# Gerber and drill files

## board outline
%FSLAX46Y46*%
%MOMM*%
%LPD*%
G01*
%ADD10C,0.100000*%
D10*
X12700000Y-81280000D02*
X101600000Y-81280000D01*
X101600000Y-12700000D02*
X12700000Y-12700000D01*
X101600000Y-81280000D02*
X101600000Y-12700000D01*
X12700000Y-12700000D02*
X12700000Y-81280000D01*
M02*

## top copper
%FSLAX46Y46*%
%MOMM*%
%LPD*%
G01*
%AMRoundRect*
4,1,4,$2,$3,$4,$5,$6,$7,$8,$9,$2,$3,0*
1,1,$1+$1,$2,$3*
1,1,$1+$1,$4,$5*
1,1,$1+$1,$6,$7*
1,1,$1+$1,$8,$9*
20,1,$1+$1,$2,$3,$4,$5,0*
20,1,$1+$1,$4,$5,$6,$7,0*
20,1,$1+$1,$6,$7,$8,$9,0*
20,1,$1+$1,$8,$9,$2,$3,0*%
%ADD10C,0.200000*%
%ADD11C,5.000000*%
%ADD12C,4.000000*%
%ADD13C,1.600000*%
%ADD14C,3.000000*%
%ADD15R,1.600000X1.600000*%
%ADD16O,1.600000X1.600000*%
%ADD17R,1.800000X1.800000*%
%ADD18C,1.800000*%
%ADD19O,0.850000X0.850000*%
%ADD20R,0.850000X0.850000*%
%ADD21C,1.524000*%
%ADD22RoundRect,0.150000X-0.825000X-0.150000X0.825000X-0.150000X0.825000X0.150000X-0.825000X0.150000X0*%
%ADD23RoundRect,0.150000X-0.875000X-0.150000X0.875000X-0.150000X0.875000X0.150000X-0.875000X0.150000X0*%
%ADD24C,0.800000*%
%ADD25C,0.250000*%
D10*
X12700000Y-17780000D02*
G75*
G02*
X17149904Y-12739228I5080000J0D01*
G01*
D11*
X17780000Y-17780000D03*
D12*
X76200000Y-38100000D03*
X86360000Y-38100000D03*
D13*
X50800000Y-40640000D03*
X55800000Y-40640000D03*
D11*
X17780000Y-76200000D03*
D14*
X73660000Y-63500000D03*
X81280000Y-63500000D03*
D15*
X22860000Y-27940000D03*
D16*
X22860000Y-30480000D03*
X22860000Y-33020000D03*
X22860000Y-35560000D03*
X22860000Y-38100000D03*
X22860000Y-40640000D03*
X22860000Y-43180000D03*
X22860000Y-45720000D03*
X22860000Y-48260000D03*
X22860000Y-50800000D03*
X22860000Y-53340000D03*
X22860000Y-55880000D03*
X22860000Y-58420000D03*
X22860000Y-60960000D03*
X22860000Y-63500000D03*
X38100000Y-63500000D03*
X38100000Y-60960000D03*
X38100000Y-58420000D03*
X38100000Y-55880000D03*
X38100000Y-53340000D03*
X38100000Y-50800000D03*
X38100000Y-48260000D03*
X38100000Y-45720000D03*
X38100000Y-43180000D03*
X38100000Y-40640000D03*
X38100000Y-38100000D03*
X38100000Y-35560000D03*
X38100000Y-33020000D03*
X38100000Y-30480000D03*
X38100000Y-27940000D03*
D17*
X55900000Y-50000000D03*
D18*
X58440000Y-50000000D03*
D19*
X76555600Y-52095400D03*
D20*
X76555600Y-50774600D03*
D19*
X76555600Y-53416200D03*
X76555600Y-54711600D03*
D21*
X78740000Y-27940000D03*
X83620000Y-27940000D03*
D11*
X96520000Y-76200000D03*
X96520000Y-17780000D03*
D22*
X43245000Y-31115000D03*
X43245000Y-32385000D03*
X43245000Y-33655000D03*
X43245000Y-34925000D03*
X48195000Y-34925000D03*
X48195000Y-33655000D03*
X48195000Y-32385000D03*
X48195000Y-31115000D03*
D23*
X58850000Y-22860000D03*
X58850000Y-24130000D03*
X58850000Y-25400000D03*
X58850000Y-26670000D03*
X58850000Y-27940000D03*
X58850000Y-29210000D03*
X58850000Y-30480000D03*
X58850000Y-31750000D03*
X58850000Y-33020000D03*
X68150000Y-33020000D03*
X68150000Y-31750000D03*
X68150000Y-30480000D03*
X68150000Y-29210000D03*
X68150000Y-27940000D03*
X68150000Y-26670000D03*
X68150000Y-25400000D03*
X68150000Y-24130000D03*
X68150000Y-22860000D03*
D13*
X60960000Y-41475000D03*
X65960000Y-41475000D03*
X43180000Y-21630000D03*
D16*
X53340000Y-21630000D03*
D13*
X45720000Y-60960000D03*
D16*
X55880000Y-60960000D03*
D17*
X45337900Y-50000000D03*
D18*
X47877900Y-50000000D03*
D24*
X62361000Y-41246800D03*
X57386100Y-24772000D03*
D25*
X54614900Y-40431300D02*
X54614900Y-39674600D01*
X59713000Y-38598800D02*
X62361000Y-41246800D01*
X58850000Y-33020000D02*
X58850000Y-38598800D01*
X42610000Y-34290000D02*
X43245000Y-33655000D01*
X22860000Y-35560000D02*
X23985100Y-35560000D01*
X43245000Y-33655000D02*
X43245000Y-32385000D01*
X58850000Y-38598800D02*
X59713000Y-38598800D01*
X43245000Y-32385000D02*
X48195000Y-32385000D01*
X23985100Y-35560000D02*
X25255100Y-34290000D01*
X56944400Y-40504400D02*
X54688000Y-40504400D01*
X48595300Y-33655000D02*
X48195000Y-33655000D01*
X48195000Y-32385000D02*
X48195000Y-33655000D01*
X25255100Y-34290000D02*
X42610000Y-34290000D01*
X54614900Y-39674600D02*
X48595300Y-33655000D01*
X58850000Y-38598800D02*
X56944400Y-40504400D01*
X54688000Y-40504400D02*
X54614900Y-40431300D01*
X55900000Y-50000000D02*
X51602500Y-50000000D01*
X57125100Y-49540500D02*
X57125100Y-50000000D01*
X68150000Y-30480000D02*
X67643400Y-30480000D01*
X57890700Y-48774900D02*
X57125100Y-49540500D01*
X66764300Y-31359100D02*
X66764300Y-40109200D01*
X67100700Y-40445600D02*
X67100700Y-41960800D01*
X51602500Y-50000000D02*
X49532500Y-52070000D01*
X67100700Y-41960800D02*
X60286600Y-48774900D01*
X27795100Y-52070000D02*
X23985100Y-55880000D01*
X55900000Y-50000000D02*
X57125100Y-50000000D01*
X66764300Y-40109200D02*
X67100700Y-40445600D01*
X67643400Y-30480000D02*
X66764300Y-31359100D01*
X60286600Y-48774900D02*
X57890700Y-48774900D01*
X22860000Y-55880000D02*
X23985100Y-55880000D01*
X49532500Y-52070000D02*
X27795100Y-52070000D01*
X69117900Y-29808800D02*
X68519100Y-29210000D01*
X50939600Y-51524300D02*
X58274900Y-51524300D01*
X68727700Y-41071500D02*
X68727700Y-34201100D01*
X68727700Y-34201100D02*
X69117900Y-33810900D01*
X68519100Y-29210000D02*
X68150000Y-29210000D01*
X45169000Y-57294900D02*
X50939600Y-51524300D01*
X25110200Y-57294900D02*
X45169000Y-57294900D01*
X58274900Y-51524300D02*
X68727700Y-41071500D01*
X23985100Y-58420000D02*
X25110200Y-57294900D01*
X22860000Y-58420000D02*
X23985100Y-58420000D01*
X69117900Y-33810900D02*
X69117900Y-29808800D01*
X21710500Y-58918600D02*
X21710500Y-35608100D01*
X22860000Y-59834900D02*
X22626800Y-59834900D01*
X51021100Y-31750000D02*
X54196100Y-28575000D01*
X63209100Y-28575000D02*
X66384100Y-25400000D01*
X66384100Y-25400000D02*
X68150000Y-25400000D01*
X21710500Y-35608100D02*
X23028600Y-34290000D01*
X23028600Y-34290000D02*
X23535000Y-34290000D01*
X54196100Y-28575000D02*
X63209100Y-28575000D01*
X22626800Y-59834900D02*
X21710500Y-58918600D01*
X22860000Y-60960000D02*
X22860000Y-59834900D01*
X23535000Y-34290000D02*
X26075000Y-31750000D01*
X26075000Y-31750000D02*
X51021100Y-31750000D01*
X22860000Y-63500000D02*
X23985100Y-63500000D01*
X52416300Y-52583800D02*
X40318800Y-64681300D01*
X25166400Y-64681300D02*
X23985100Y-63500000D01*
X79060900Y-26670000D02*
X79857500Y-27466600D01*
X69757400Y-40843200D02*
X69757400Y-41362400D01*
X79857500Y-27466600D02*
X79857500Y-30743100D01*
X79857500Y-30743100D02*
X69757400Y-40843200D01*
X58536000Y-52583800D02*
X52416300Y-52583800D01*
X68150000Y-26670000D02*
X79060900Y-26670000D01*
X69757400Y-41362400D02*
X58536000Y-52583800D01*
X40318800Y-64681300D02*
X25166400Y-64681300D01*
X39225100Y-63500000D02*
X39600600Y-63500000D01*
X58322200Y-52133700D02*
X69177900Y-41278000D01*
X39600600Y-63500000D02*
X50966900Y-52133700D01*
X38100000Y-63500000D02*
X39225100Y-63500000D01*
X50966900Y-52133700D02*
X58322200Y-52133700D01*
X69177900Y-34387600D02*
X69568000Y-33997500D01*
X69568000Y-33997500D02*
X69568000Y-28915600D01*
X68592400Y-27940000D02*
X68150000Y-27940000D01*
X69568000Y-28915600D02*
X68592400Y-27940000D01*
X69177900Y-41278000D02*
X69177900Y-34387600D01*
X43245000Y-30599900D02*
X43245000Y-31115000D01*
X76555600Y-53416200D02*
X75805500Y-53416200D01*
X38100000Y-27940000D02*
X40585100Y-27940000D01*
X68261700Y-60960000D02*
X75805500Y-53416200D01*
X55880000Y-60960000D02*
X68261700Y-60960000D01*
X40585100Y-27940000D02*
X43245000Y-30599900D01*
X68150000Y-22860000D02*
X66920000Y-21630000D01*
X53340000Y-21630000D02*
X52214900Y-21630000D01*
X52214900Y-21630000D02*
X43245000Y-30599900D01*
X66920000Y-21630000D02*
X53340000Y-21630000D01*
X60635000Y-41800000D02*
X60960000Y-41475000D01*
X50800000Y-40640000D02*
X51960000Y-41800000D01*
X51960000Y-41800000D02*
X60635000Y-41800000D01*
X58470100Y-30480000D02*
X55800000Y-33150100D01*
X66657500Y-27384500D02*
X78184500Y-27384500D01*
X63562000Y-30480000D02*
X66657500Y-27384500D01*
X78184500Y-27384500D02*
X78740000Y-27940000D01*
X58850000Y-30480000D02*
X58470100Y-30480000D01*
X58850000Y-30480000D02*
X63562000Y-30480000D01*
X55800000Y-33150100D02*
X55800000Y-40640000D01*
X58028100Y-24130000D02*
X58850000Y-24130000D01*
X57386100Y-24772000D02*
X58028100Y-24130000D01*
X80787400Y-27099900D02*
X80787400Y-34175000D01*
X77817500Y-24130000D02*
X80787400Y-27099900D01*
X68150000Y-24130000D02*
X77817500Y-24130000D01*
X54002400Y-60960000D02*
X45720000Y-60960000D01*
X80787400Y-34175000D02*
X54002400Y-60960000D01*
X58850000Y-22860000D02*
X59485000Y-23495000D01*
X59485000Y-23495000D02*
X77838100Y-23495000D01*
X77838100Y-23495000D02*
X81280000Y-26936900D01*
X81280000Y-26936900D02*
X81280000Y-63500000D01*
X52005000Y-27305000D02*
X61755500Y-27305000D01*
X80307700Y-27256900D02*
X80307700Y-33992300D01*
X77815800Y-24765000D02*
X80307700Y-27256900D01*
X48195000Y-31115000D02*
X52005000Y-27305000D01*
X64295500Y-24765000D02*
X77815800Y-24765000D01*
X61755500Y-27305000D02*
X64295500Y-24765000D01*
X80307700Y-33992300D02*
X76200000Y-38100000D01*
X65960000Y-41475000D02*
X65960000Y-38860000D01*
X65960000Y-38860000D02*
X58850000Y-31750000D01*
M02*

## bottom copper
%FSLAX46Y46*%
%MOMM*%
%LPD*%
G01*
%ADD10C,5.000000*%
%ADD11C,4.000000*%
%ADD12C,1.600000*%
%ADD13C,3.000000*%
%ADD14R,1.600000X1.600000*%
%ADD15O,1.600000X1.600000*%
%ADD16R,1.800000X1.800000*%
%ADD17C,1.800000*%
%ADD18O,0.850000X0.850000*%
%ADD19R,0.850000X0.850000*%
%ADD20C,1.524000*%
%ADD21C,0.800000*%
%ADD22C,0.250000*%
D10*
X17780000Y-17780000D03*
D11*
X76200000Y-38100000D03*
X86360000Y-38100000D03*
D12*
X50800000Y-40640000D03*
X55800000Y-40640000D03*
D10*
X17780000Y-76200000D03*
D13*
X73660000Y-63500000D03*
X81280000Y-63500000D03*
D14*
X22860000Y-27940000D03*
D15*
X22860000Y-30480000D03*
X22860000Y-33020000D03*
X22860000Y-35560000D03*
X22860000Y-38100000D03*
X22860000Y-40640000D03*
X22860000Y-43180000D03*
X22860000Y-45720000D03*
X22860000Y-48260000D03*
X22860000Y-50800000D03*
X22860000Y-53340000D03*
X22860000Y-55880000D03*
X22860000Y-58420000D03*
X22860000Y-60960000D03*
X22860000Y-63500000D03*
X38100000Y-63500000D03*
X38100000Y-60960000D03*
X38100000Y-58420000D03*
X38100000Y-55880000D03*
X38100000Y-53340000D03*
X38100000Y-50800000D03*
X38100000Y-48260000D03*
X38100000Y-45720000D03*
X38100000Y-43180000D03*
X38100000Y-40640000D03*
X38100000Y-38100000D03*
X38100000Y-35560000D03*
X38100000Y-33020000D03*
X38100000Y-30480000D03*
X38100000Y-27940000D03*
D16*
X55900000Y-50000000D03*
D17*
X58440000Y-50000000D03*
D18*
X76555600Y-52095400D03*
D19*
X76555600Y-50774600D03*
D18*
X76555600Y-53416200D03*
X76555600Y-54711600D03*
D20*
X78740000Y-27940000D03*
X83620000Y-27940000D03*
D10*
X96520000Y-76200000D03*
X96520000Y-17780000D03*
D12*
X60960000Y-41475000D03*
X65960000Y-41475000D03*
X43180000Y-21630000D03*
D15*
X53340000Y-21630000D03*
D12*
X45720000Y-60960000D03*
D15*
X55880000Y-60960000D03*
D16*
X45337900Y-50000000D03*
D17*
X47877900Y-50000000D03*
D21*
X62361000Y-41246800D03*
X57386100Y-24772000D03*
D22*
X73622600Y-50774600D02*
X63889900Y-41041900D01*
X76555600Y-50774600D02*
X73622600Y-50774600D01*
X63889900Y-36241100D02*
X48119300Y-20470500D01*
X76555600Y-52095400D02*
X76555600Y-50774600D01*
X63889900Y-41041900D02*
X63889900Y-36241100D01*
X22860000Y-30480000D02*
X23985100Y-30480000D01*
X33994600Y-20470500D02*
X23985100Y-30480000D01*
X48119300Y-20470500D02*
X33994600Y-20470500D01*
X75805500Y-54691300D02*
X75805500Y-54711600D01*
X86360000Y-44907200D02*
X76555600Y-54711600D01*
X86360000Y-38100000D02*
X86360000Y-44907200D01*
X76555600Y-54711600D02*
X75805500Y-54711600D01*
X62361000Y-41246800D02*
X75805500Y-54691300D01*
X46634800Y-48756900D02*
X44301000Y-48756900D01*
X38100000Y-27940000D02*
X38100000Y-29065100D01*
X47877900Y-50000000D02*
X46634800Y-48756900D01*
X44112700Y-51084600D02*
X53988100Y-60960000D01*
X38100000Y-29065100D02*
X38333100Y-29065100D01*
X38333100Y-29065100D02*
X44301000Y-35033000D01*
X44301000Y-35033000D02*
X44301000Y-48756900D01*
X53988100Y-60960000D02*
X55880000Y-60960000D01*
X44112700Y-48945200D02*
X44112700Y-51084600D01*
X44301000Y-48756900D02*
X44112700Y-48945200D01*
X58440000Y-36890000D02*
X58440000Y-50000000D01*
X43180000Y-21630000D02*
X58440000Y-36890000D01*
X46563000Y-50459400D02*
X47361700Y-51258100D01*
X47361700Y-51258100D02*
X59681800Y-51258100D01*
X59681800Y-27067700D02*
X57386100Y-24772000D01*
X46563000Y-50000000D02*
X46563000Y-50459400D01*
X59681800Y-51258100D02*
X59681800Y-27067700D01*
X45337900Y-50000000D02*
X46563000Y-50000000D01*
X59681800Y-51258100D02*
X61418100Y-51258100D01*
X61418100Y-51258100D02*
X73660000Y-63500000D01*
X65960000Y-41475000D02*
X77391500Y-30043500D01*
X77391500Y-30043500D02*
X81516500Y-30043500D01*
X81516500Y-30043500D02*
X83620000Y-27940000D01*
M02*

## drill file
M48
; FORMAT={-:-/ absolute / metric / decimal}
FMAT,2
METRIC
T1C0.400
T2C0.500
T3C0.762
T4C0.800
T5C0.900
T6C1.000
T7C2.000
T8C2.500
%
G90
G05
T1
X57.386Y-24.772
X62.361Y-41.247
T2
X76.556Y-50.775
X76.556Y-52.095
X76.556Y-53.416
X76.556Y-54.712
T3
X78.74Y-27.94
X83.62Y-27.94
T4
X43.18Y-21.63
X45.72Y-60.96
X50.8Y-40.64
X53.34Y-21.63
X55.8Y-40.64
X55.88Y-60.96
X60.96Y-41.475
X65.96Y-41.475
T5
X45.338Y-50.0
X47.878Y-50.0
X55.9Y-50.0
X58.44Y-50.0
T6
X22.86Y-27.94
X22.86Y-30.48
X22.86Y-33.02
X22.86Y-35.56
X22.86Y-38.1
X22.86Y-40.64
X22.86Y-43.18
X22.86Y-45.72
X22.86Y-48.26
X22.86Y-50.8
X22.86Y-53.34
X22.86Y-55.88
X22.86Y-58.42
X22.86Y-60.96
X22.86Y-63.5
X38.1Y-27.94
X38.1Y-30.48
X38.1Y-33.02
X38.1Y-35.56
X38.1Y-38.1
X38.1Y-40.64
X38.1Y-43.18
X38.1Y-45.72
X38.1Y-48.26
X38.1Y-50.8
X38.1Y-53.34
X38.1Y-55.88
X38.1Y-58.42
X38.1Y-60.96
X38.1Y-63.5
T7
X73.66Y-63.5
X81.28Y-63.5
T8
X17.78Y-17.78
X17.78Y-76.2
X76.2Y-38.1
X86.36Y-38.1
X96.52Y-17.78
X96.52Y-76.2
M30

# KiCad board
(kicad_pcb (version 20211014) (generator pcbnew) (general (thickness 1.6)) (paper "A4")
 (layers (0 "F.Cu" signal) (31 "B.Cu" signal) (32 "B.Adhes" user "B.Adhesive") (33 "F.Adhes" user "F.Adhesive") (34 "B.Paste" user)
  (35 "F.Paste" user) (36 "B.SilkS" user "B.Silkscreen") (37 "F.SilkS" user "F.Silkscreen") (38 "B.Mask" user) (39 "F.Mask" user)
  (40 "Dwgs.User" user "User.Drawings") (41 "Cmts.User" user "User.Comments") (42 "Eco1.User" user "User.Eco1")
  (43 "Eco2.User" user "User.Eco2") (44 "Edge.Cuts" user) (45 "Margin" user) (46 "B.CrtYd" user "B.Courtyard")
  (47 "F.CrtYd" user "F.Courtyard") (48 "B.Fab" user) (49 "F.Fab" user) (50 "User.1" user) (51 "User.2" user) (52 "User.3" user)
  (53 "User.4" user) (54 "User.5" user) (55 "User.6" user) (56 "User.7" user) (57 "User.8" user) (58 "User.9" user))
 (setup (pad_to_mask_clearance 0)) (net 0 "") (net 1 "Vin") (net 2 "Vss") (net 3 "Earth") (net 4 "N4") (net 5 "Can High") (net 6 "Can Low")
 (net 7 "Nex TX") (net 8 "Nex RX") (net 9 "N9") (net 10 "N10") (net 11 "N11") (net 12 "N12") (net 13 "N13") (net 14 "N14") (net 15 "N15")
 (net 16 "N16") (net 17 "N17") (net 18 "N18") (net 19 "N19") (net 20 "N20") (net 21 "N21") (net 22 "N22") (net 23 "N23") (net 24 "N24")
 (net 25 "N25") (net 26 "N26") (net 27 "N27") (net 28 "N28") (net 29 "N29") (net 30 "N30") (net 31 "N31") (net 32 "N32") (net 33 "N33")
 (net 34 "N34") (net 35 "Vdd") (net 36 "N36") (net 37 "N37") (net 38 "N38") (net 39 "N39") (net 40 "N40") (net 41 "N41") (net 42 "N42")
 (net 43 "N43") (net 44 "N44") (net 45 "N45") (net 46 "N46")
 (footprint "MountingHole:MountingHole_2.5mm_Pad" (layer "F.Cu") (at 17.78 17.78)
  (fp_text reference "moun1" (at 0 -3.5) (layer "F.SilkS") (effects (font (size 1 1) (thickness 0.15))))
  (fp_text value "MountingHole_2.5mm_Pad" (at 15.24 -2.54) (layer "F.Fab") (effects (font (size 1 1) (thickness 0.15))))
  (pad "1" thru_hole circle (at 0 0) (size 5 5) (drill 2.5) (layers *.Cu *.Mask)))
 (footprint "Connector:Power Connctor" (layer "F.Cu") (at 76.2 33.02)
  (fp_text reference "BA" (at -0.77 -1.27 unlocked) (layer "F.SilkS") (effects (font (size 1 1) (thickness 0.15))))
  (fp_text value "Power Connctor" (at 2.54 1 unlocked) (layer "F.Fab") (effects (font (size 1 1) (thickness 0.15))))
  (pad "1" thru_hole circle (at 0 5.08) (size 4 4) (drill 2.5) (layers *.Cu *.Mask) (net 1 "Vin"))
  (pad "2" thru_hole circle (at 10.16 5.08) (size 4 4) (drill 2.5) (layers *.Cu *.Mask) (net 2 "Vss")))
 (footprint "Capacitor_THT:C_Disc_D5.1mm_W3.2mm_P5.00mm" (layer "F.Cu") (at 50.8 40.64)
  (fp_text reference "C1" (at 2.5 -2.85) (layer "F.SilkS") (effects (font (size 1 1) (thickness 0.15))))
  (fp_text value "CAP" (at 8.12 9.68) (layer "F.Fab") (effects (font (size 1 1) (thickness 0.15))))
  (pad "1" thru_hole circle (at 0 0) (size 1.6 1.6) (drill 0.8) (layers *.Cu *.Mask) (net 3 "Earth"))
  (pad "2" thru_hole circle (at 5 0) (size 1.6 1.6) (drill 0.8) (layers *.Cu *.Mask) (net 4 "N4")))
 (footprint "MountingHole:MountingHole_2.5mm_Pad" (layer "F.Cu") (at 17.78 76.2)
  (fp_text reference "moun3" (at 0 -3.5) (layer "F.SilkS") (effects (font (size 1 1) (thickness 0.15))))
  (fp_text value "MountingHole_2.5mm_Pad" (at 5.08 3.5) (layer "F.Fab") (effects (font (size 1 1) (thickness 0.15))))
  (pad "1" thru_hole circle (at 0 0) (size 5 5) (drill 2.5) (layers *.Cu *.Mask)))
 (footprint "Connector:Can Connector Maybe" (layer "F.Cu") (at 76.2 58.42)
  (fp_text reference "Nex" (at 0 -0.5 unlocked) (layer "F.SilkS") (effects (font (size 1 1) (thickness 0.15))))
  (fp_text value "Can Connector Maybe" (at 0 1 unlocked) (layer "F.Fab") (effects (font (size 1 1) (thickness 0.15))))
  (pad "1" thru_hole circle (at -2.54 5.08) (size 3 3) (drill 2) (layers *.Cu *.Mask) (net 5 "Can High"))
  (pad "2" thru_hole circle (at 5.08 5.08) (size 3 3) (drill 2) (layers *.Cu *.Mask) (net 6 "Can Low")))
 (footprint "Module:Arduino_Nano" (layer "F.Cu") (at 22.86 27.94)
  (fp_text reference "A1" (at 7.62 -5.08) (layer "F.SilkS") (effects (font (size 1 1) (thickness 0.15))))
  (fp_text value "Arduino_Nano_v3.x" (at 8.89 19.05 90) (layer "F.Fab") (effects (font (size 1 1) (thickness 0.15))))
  (pad "1" thru_hole rect (at 0 0) (size 1.6 1.6) (drill 1) (layers *.Cu *.Mask) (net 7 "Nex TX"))
  (pad "2" thru_hole oval (at 0 2.54) (size 1.6 1.6) (drill 1) (layers *.Cu *.Mask) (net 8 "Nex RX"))
  (pad "3" thru_hole oval (at 0 5.08) (size 1.6 1.6) (drill 1) (layers *.Cu *.Mask) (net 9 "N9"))
  (pad "4" thru_hole oval (at 0 7.62) (size 1.6 1.6) (drill 1) (layers *.Cu *.Mask) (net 2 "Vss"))
  (pad "5" thru_hole oval (at 0 10.16) (size 1.6 1.6) (drill 1) (layers *.Cu *.Mask) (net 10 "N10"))
  (pad "6" thru_hole oval (at 0 12.7) (size 1.6 1.6) (drill 1) (layers *.Cu *.Mask) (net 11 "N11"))
  (pad "7" thru_hole oval (at 0 15.24) (size 1.6 1.6) (drill 1) (layers *.Cu *.Mask) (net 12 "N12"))
  (pad "8" thru_hole oval (at 0 17.78) (size 1.6 1.6) (drill 1) (layers *.Cu *.Mask) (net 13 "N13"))
  (pad "9" thru_hole oval (at 0 20.32) (size 1.6 1.6) (drill 1) (layers *.Cu *.Mask) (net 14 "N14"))
  (pad "10" thru_hole oval (at 0 22.86) (size 1.6 1.6) (drill 1) (layers *.Cu *.Mask) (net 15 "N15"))
  (pad "11" thru_hole oval (at 0 25.4) (size 1.6 1.6) (drill 1) (layers *.Cu *.Mask) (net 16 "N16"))
  (pad "12" thru_hole oval (at 0 27.94) (size 1.6 1.6) (drill 1) (layers *.Cu *.Mask) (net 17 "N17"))
  (pad "13" thru_hole oval (at 0 30.48) (size 1.6 1.6) (drill 1) (layers *.Cu *.Mask) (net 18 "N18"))
  (pad "14" thru_hole oval (at 0 33.02) (size 1.6 1.6) (drill 1) (layers *.Cu *.Mask) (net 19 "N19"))
  (pad "15" thru_hole oval (at 0 35.56) (size 1.6 1.6) (drill 1) (layers *.Cu *.Mask) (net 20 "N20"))
  (pad "16" thru_hole oval (at 15.24 35.56) (size 1.6 1.6) (drill 1) (layers *.Cu *.Mask) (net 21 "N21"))
  (pad "17" thru_hole oval (at 15.24 33.02) (size 1.6 1.6) (drill 1) (layers *.Cu *.Mask) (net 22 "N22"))
  (pad "18" thru_hole oval (at 15.24 30.48) (size 1.6 1.6) (drill 1) (layers *.Cu *.Mask) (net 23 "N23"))
  (pad "19" thru_hole oval (at 15.24 27.94) (size 1.6 1.6) (drill 1) (layers *.Cu *.Mask) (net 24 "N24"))
  (pad "20" thru_hole oval (at 15.24 25.4) (size 1.6 1.6) (drill 1) (layers *.Cu *.Mask) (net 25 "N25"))
  (pad "21" thru_hole oval (at 15.24 22.86) (size 1.6 1.6) (drill 1) (layers *.Cu *.Mask) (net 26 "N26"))
  (pad "22" thru_hole oval (at 15.24 20.32) (size 1.6 1.6) (drill 1) (layers *.Cu *.Mask) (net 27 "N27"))
  (pad "23" thru_hole oval (at 15.24 17.78) (size 1.6 1.6) (drill 1) (layers *.Cu *.Mask) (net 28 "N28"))
  (pad "24" thru_hole oval (at 15.24 15.24) (size 1.6 1.6) (drill 1) (layers *.Cu *.Mask) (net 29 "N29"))
  (pad "25" thru_hole oval (at 15.24 12.7) (size 1.6 1.6) (drill 1) (layers *.Cu *.Mask) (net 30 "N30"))
  (pad "26" thru_hole oval (at 15.24 10.16) (size 1.6 1.6) (drill 1) (layers *.Cu *.Mask) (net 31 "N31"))
  (pad "27" thru_hole oval (at 15.24 7.62) (size 1.6 1.6) (drill 1) (layers *.Cu *.Mask) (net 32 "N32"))
  (pad "28" thru_hole oval (at 15.24 5.08) (size 1.6 1.6) (drill 1) (layers *.Cu *.Mask) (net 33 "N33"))
  (pad "29" thru_hole oval (at 15.24 2.54) (size 1.6 1.6) (drill 1) (layers *.Cu *.Mask) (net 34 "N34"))
  (pad "30" thru_hole oval (at 15.24 0) (size 1.6 1.6) (drill 1) (layers *.Cu *.Mask) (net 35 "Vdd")))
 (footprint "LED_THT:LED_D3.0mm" (layer "F.Cu") (at 55.9 50)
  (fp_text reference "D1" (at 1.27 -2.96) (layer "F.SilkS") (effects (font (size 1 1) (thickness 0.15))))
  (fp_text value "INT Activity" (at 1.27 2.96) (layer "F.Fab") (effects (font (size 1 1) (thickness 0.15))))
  (pad "1" thru_hole rect (at 0 0) (size 1.8 1.8) (drill 0.9) (layers *.Cu *.Mask) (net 17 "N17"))
  (pad "2" thru_hole circle (at 2.54 0) (size 1.8 1.8) (drill 0.9) (layers *.Cu *.Mask) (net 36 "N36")))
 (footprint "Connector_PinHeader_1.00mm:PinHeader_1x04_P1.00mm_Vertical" (layer "F.Cu") (at 76.2 50.8)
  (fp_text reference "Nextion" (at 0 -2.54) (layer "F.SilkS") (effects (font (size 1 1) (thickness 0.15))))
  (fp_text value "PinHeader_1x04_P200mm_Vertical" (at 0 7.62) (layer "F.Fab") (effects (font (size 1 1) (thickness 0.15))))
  (pad "2" thru_hole oval (at 0.3556 1.2954) (size 0.85 0.85) (drill 0.5) (layers *.Cu *.Mask) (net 8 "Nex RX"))
  (pad "2" thru_hole rect (at 0.3556 -0.0254) (size 0.85 0.85) (drill 0.5) (layers *.Cu *.Mask) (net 8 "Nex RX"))
  (pad "3" thru_hole oval (at 0.3556 2.6162) (size 0.85 0.85) (drill 0.5) (layers *.Cu *.Mask) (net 35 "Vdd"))
  (pad "4" thru_hole oval (at 0.3556 3.9116) (size 0.85 0.85) (drill 0.5) (layers *.Cu *.Mask) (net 2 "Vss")))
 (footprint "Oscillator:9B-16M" (layer "F.Cu") (at 78.74 27.94)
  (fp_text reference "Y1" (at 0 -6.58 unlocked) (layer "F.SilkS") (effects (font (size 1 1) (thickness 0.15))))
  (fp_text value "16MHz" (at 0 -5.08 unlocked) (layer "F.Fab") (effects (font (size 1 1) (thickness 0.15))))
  (pad "1" thru_hole circle (at 0 0) (size 1.524 1.524) (drill 0.762) (layers *.Cu *.Mask) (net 4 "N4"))
  (pad "2" thru_hole circle (at 4.88 0) (size 1.524 1.524) (drill 0.762) (layers *.Cu *.Mask) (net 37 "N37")))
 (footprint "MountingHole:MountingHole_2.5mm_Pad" (layer "F.Cu") (at 96.52 76.2)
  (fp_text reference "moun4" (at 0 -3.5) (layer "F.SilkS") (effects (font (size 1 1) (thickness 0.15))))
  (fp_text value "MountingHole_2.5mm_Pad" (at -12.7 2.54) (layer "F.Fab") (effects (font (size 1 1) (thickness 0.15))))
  (pad "1" thru_hole circle (at 0 0) (size 5 5) (drill 2.5) (layers *.Cu *.Mask)))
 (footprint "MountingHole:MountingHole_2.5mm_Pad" (layer "F.Cu") (at 96.52 17.78)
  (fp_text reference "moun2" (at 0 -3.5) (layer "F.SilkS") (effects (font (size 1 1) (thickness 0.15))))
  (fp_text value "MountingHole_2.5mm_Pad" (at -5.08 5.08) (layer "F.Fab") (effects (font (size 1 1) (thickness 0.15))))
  (pad "1" thru_hole circle (at 0 0) (size 5 5) (drill 2.5) (layers *.Cu *.Mask)))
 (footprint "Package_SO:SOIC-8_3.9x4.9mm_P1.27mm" (layer "F.Cu") (at 45.72 33.02)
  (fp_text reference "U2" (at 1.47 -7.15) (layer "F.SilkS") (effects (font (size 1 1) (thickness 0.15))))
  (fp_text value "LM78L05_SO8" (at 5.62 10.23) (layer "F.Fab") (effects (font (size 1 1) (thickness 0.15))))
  (pad "1" smd roundrect (at -2.475 -1.905) (size 1.95 0.6) (layers "F.Cu" "F.Paste" "F.Mask") (roundrect_rratio 0.25) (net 35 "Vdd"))
  (pad "2" smd roundrect (at -2.475 -0.635) (size 1.95 0.6) (layers "F.Cu" "F.Paste" "F.Mask") (roundrect_rratio 0.25) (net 2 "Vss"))
  (pad "3" smd roundrect (at -2.475 0.635) (size 1.95 0.6) (layers "F.Cu" "F.Paste" "F.Mask") (roundrect_rratio 0.25) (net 2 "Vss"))
  (pad "4" smd roundrect (at -2.475 1.905) (size 1.95 0.6) (layers "F.Cu" "F.Paste" "F.Mask") (roundrect_rratio 0.25) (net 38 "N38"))
  (pad "5" smd roundrect (at 2.475 1.905) (size 1.95 0.6) (layers "F.Cu" "F.Paste" "F.Mask") (roundrect_rratio 0.25) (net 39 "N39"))
  (pad "6" smd roundrect (at 2.475 0.635) (size 1.95 0.6) (layers "F.Cu" "F.Paste" "F.Mask") (roundrect_rratio 0.25) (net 2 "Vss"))
  (pad "7" smd roundrect (at 2.475 -0.635) (size 1.95 0.6) (layers "F.Cu" "F.Paste" "F.Mask") (roundrect_rratio 0.25) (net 2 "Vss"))
  (pad "8" smd roundrect (at 2.475 -1.905) (size 1.95 0.6) (layers "F.Cu" "F.Paste" "F.Mask") (roundrect_rratio 0.25) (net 1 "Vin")))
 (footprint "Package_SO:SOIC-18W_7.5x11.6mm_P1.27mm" (layer "F.Cu") (at 63.5 27.94)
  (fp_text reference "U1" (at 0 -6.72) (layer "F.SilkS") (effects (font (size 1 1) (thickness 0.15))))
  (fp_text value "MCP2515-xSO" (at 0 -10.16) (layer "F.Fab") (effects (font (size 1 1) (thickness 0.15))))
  (pad "1" smd roundrect (at -4.65 -5.08) (size 2.05 0.6) (layers "F.Cu" "F.Paste" "F.Mask") (roundrect_rratio 0.25) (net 6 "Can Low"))
  (pad "2" smd roundrect (at -4.65 -3.81) (size 2.05 0.6) (layers "F.Cu" "F.Paste" "F.Mask") (roundrect_rratio 0.25) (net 5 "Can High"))
  (pad "3" smd roundrect (at -4.65 -2.54) (size 2.05 0.6) (layers "F.Cu" "F.Paste" "F.Mask") (roundrect_rratio 0.25) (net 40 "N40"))
  (pad "4" smd roundrect (at -4.65 -1.27) (size 2.05 0.6) (layers "F.Cu" "F.Paste" "F.Mask") (roundrect_rratio 0.25) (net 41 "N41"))
  (pad "5" smd roundrect (at -4.65 0) (size 2.05 0.6) (layers "F.Cu" "F.Paste" "F.Mask") (roundrect_rratio 0.25) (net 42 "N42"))
  (pad "6" smd roundrect (at -4.65 1.27) (size 2.05 0.6) (layers "F.Cu" "F.Paste" "F.Mask") (roundrect_rratio 0.25) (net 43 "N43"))
  (pad "7" smd roundrect (at -4.65 2.54) (size 2.05 0.6) (layers "F.Cu" "F.Paste" "F.Mask") (roundrect_rratio 0.25) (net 4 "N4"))
  (pad "8" smd roundrect (at -4.65 3.81) (size 2.05 0.6) (layers "F.Cu" "F.Paste" "F.Mask") (roundrect_rratio 0.25) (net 37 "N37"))
  (pad "9" smd roundrect (at -4.65 5.08) (size 2.05 0.6) (layers "F.Cu" "F.Paste" "F.Mask") (roundrect_rratio 0.25) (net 2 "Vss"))
  (pad "10" smd roundrect (at 4.65 5.08) (size 2.05 0.6) (layers "F.Cu" "F.Paste" "F.Mask") (roundrect_rratio 0.25) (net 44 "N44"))
  (pad "11" smd roundrect (at 4.65 3.81) (size 2.05 0.6) (layers "F.Cu" "F.Paste" "F.Mask") (roundrect_rratio 0.25) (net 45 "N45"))
  (pad "12" smd roundrect (at 4.65 2.54) (size 2.05 0.6) (layers "F.Cu" "F.Paste" "F.Mask") (roundrect_rratio 0.25) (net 17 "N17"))
  (pad "13" smd roundrect (at 4.65 1.27) (size 2.05 0.6) (layers "F.Cu" "F.Paste" "F.Mask") (roundrect_rratio 0.25) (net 18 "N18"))
  (pad "14" smd roundrect (at 4.65 0) (size 2.05 0.6) (layers "F.Cu" "F.Paste" "F.Mask") (roundrect_rratio 0.25) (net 21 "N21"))
  (pad "15" smd roundrect (at 4.65 -1.27) (size 2.05 0.6) (layers "F.Cu" "F.Paste" "F.Mask") (roundrect_rratio 0.25) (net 20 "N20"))
  (pad "16" smd roundrect (at 4.65 -2.54) (size 2.05 0.6) (layers "F.Cu" "F.Paste" "F.Mask") (roundrect_rratio 0.25) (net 19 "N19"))
  (pad "17" smd roundrect (at 4.65 -3.81) (size 2.05 0.6) (layers "F.Cu" "F.Paste" "F.Mask") (roundrect_rratio 0.25) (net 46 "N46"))
  (pad "18" smd roundrect (at 4.65 -5.08) (size 2.05 0.6) (layers "F.Cu" "F.Paste" "F.Mask") (roundrect_rratio 0.25) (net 35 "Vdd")))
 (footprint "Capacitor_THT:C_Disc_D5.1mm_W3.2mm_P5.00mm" (layer "F.Cu") (at 60.96 41.475)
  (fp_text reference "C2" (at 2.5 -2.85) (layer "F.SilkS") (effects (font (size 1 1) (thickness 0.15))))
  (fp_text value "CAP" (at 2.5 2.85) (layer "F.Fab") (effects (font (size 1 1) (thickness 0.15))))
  (pad "1" thru_hole circle (at 0 0) (size 1.6 1.6) (drill 0.8) (layers *.Cu *.Mask) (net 3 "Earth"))
  (pad "2" thru_hole circle (at 5 0) (size 1.6 1.6) (drill 0.8) (layers *.Cu *.Mask) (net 37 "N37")))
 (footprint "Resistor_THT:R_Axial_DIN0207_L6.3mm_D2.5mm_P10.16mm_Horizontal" (layer "F.Cu") (at 43.18 21.63)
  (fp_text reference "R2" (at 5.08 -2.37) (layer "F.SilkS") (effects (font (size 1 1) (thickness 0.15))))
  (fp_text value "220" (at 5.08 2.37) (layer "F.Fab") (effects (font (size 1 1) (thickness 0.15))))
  (pad "1" thru_hole circle (at 0 0) (size 1.6 1.6) (drill 0.8) (layers *.Cu *.Mask) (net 36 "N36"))
  (pad "2" thru_hole oval (at 10.16 0) (size 1.6 1.6) (drill 0.8) (layers *.Cu *.Mask) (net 35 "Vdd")))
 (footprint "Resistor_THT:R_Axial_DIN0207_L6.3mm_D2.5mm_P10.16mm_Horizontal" (layer "F.Cu") (at 45.72 60.96)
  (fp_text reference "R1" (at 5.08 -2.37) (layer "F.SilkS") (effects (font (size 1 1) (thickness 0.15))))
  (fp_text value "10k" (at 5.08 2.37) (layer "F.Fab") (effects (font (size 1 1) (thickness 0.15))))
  (pad "1" thru_hole circle (at 0 0) (size 1.6 1.6) (drill 0.8) (layers *.Cu *.Mask) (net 46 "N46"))
  (pad "2" thru_hole oval (at 10.16 0) (size 1.6 1.6) (drill 0.8) (layers *.Cu *.Mask) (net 35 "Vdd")))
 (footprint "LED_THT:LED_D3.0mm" (layer "F.Cu") (at 45.3379 50)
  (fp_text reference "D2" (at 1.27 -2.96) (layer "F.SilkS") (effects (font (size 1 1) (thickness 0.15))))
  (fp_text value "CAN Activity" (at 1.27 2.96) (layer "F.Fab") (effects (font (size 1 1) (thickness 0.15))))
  (pad "1" thru_hole rect (at 0 0) (size 1.8 1.8) (drill 0.9) (layers *.Cu *.Mask) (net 5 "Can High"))
  (pad "2" thru_hole circle (at 2.54 0) (size 1.8 1.8) (drill 0.9) (layers *.Cu *.Mask) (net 35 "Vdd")))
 (gr_arc (start 12.7 17.78) (mid 13.971635 14.418043) (end 17.149904 12.739228) (layer "F.Cu") (width 0.2))
 (gr_line (start 12.7 81.28) (end 101.6 81.28) (layer "Edge.Cuts") (width 0.1))
 (gr_line (start 101.6 12.7) (end 12.7 12.7) (layer "Edge.Cuts") (width 0.1))
 (gr_line (start 101.6 81.28) (end 101.6 12.7) (layer "Edge.Cuts") (width 0.1))
 (gr_line (start 12.7 12.7) (end 12.7 81.28) (layer "Edge.Cuts") (width 0.1))
 (segment (start 73.6226 50.7746) (end 63.8899 41.0419) (width 0.25) (layer "B.Cu") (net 8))
 (segment (start 76.5556 50.7746) (end 73.6226 50.7746) (width 0.25) (layer "B.Cu") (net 8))
 (segment (start 63.8899 36.2411) (end 48.1193 20.4705) (width 0.25) (layer "B.Cu") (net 8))
 (segment (start 76.5556 52.0954) (end 76.5556 50.7746) (width 0.25) (layer "B.Cu") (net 8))
 (segment (start 63.8899 41.0419) (end 63.8899 36.2411) (width 0.25) (layer "B.Cu") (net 8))
 (segment (start 22.86 30.48) (end 23.9851 30.48) (width 0.25) (layer "B.Cu") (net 8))
 (segment (start 33.9946 20.4705) (end 23.9851 30.48) (width 0.25) (layer "B.Cu") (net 8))
 (segment (start 48.1193 20.4705) (end 33.9946 20.4705) (width 0.25) (layer "B.Cu") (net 8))
 (segment (start 54.6149 40.4313) (end 54.6149 39.6746) (width 0.25) (layer "F.Cu") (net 2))
 (segment (start 59.713 38.5988) (end 62.361 41.2468) (width 0.25) (layer "F.Cu") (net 2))
 (segment (start 58.85 33.02) (end 58.85 38.5988) (width 0.25) (layer "F.Cu") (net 2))
 (segment (start 42.61 34.29) (end 43.245 33.655) (width 0.25) (layer "F.Cu") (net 2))
 (segment (start 22.86 35.56) (end 23.9851 35.56) (width 0.25) (layer "F.Cu") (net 2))
 (segment (start 43.245 33.655) (end 43.245 32.385) (width 0.25) (layer "F.Cu") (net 2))
 (segment (start 58.85 38.5988) (end 59.713 38.5988) (width 0.25) (layer "F.Cu") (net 2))
 (segment (start 43.245 32.385) (end 48.195 32.385) (width 0.25) (layer "F.Cu") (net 2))
 (segment (start 23.9851 35.56) (end 25.2551 34.29) (width 0.25) (layer "F.Cu") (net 2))
 (segment (start 56.9444 40.5044) (end 54.688 40.5044) (width 0.25) (layer "F.Cu") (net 2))
 (segment (start 48.5953 33.655) (end 48.195 33.655) (width 0.25) (layer "F.Cu") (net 2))
 (segment (start 48.195 32.385) (end 48.195 33.655) (width 0.25) (layer "F.Cu") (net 2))
 (segment (start 25.2551 34.29) (end 42.61 34.29) (width 0.25) (layer "F.Cu") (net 2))
 (segment (start 54.6149 39.6746) (end 48.5953 33.655) (width 0.25) (layer "F.Cu") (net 2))
 (segment (start 58.85 38.5988) (end 56.9444 40.5044) (width 0.25) (layer "F.Cu") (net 2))
 (segment (start 54.688 40.5044) (end 54.6149 40.4313) (width 0.25) (layer "F.Cu") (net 2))
 (via (at 62.361 41.2468) (size 0.8) (drill 0.4) (layers "F.Cu" "B.Cu") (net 2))
 (segment (start 75.8055 54.6913) (end 75.8055 54.7116) (width 0.25) (layer "B.Cu") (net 2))
 (segment (start 86.36 44.9072) (end 76.5556 54.7116) (width 0.25) (layer "B.Cu") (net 2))
 (segment (start 86.36 38.1) (end 86.36 44.9072) (width 0.25) (layer "B.Cu") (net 2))
 (segment (start 76.5556 54.7116) (end 75.8055 54.7116) (width 0.25) (layer "B.Cu") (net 2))
 (segment (start 62.361 41.2468) (end 75.8055 54.6913) (width 0.25) (layer "B.Cu") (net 2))
 (segment (start 55.9 50) (end 51.6025 50) (width 0.25) (layer "F.Cu") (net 17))
 (segment (start 57.1251 49.5405) (end 57.1251 50) (width 0.25) (layer "F.Cu") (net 17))
 (segment (start 68.15 30.48) (end 67.6434 30.48) (width 0.25) (layer "F.Cu") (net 17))
 (segment (start 57.8907 48.7749) (end 57.1251 49.5405) (width 0.25) (layer "F.Cu") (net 17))
 (segment (start 66.7643 31.3591) (end 66.7643 40.1092) (width 0.25) (layer "F.Cu") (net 17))
 (segment (start 67.1007 40.4456) (end 67.1007 41.9608) (width 0.25) (layer "F.Cu") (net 17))
 (segment (start 51.6025 50) (end 49.5325 52.07) (width 0.25) (layer "F.Cu") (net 17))
 (segment (start 67.1007 41.9608) (end 60.2866 48.7749) (width 0.25) (layer "F.Cu") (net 17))
 (segment (start 27.7951 52.07) (end 23.9851 55.88) (width 0.25) (layer "F.Cu") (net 17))
 (segment (start 55.9 50) (end 57.1251 50) (width 0.25) (layer "F.Cu") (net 17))
 (segment (start 66.7643 40.1092) (end 67.1007 40.4456) (width 0.25) (layer "F.Cu") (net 17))
 (segment (start 67.6434 30.48) (end 66.7643 31.3591) (width 0.25) (layer "F.Cu") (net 17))
 (segment (start 60.2866 48.7749) (end 57.8907 48.7749) (width 0.25) (layer "F.Cu") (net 17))
 (segment (start 22.86 55.88) (end 23.9851 55.88) (width 0.25) (layer "F.Cu") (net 17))
 (segment (start 49.5325 52.07) (end 27.7951 52.07) (width 0.25) (layer "F.Cu") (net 17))
 (segment (start 69.1179 29.8088) (end 68.5191 29.21) (width 0.25) (layer "F.Cu") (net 18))
 (segment (start 50.9396 51.5243) (end 58.2749 51.5243) (width 0.25) (layer "F.Cu") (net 18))
 (segment (start 68.7277 41.0715) (end 68.7277 34.2011) (width 0.25) (layer "F.Cu") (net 18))
 (segment (start 68.7277 34.2011) (end 69.1179 33.8109) (width 0.25) (layer "F.Cu") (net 18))
 (segment (start 68.5191 29.21) (end 68.15 29.21) (width 0.25) (layer "F.Cu") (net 18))
 (segment (start 45.169 57.2949) (end 50.9396 51.5243) (width 0.25) (layer "F.Cu") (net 18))
 (segment (start 25.1102 57.2949) (end 45.169 57.2949) (width 0.25) (layer "F.Cu") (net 18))
 (segment (start 58.2749 51.5243) (end 68.7277 41.0715) (width 0.25) (layer "F.Cu") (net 18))
 (segment (start 23.9851 58.42) (end 25.1102 57.2949) (width 0.25) (layer "F.Cu") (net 18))
 (segment (start 22.86 58.42) (end 23.9851 58.42) (width 0.25) (layer "F.Cu") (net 18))
 (segment (start 69.1179 33.8109) (end 69.1179 29.8088) (width 0.25) (layer "F.Cu") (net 18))
 (segment (start 21.7105 58.9186) (end 21.7105 35.6081) (width 0.25) (layer "F.Cu") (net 19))
 (segment (start 22.86 59.8349) (end 22.6268 59.8349) (width 0.25) (layer "F.Cu") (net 19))
 (segment (start 51.0211 31.75) (end 54.1961 28.575) (width 0.25) (layer "F.Cu") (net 19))
 (segment (start 63.2091 28.575) (end 66.3841 25.4) (width 0.25) (layer "F.Cu") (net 19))
 (segment (start 66.3841 25.4) (end 68.15 25.4) (width 0.25) (layer "F.Cu") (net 19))
 (segment (start 21.7105 35.6081) (end 23.0286 34.29) (width 0.25) (layer "F.Cu") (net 19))
 (segment (start 23.0286 34.29) (end 23.535 34.29) (width 0.25) (layer "F.Cu") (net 19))
 (segment (start 54.1961 28.575) (end 63.2091 28.575) (width 0.25) (layer "F.Cu") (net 19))
 (segment (start 22.6268 59.8349) (end 21.7105 58.9186) (width 0.25) (layer "F.Cu") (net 19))
 (segment (start 22.86 60.96) (end 22.86 59.8349) (width 0.25) (layer "F.Cu") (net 19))
 (segment (start 23.535 34.29) (end 26.075 31.75) (width 0.25) (layer "F.Cu") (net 19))
 (segment (start 26.075 31.75) (end 51.0211 31.75) (width 0.25) (layer "F.Cu") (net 19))
 (segment (start 22.86 63.5) (end 23.9851 63.5) (width 0.25) (layer "F.Cu") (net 20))
 (segment (start 52.4163 52.5838) (end 40.3188 64.6813) (width 0.25) (layer "F.Cu") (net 20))
 (segment (start 25.1664 64.6813) (end 23.9851 63.5) (width 0.25) (layer "F.Cu") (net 20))
 (segment (start 79.0609 26.67) (end 79.8575 27.4666) (width 0.25) (layer "F.Cu") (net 20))
 (segment (start 69.7574 40.8432) (end 69.7574 41.3624) (width 0.25) (layer "F.Cu") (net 20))
 (segment (start 79.8575 27.4666) (end 79.8575 30.7431) (width 0.25) (layer "F.Cu") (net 20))
 (segment (start 79.8575 30.7431) (end 69.7574 40.8432) (width 0.25) (layer "F.Cu") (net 20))
 (segment (start 58.536 52.5838) (end 52.4163 52.5838) (width 0.25) (layer "F.Cu") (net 20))
 (segment (start 68.15 26.67) (end 79.0609 26.67) (width 0.25) (layer "F.Cu") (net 20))
 (segment (start 69.7574 41.3624) (end 58.536 52.5838) (width 0.25) (layer "F.Cu") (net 20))
 (segment (start 40.3188 64.6813) (end 25.1664 64.6813) (width 0.25) (layer "F.Cu") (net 20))
 (segment (start 39.2251 63.5) (end 39.6006 63.5) (width 0.25) (layer "F.Cu") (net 21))
 (segment (start 58.3222 52.1337) (end 69.1779 41.278) (width 0.25) (layer "F.Cu") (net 21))
 (segment (start 39.6006 63.5) (end 50.9669 52.1337) (width 0.25) (layer "F.Cu") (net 21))
 (segment (start 38.1 63.5) (end 39.2251 63.5) (width 0.25) (layer "F.Cu") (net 21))
 (segment (start 50.9669 52.1337) (end 58.3222 52.1337) (width 0.25) (layer "F.Cu") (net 21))
 (segment (start 69.1779 34.3876) (end 69.568 33.9975) (width 0.25) (layer "F.Cu") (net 21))
 (segment (start 69.568 33.9975) (end 69.568 28.9156) (width 0.25) (layer "F.Cu") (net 21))
 (segment (start 68.5924 27.94) (end 68.15 27.94) (width 0.25) (layer "F.Cu") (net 21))
 (segment (start 69.568 28.9156) (end 68.5924 27.94) (width 0.25) (layer "F.Cu") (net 21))
 (segment (start 69.1779 41.278) (end 69.1779 34.3876) (width 0.25) (layer "F.Cu") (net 21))
 (segment (start 43.245 30.5999) (end 43.245 31.115) (width 0.25) (layer "F.Cu") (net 35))
 (segment (start 76.5556 53.4162) (end 75.8055 53.4162) (width 0.25) (layer "F.Cu") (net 35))
 (segment (start 38.1 27.94) (end 40.5851 27.94) (width 0.25) (layer "F.Cu") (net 35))
 (segment (start 68.2617 60.96) (end 75.8055 53.4162) (width 0.25) (layer "F.Cu") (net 35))
 (segment (start 55.88 60.96) (end 68.2617 60.96) (width 0.25) (layer "F.Cu") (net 35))
 (segment (start 40.5851 27.94) (end 43.245 30.5999) (width 0.25) (layer "F.Cu") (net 35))
 (segment (start 68.15 22.86) (end 66.92 21.63) (width 0.25) (layer "F.Cu") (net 35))
 (segment (start 53.34 21.63) (end 52.2149 21.63) (width 0.25) (layer "F.Cu") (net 35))
 (segment (start 52.2149 21.63) (end 43.245 30.5999) (width 0.25) (layer "F.Cu") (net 35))
 (segment (start 66.92 21.63) (end 53.34 21.63) (width 0.25) (layer "F.Cu") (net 35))
 (segment (start 46.6348 48.7569) (end 44.301 48.7569) (width 0.25) (layer "B.Cu") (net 35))
 (segment (start 38.1 27.94) (end 38.1 29.0651) (width 0.25) (layer "B.Cu") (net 35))
 (segment (start 47.8779 50) (end 46.6348 48.7569) (width 0.25) (layer "B.Cu") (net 35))
 (segment (start 44.1127 51.0846) (end 53.9881 60.96) (width 0.25) (layer "B.Cu") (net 35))
 (segment (start 38.1 29.0651) (end 38.3331 29.0651) (width 0.25) (layer "B.Cu") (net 35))
 (segment (start 38.3331 29.0651) (end 44.301 35.033) (width 0.25) (layer "B.Cu") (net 35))
 (segment (start 44.301 35.033) (end 44.301 48.7569) (width 0.25) (layer "B.Cu") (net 35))
 (segment (start 53.9881 60.96) (end 55.88 60.96) (width 0.25) (layer "B.Cu") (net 35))
 (segment (start 44.1127 48.9452) (end 44.1127 51.0846) (width 0.25) (layer "B.Cu") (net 35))
 (segment (start 44.301 48.7569) (end 44.1127 48.9452) (width 0.25) (layer "B.Cu") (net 35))
 (segment (start 60.635 41.8) (end 60.96 41.475) (width 0.25) (layer "F.Cu") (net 3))
 (segment (start 50.8 40.64) (end 51.96 41.8) (width 0.25) (layer "F.Cu") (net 3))
 (segment (start 51.96 41.8) (end 60.635 41.8) (width 0.25) (layer "F.Cu") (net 3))
 (segment (start 58.4701 30.48) (end 55.8 33.1501) (width 0.25) (layer "F.Cu") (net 4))
 (segment (start 66.6575 27.3845) (end 78.1845 27.3845) (width 0.25) (layer "F.Cu") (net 4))
 (segment (start 63.562 30.48) (end 66.6575 27.3845) (width 0.25) (layer "F.Cu") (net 4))
 (segment (start 78.1845 27.3845) (end 78.74 27.94) (width 0.25) (layer "F.Cu") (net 4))
 (segment (start 58.85 30.48) (end 58.4701 30.48) (width 0.25) (layer "F.Cu") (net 4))
 (segment (start 58.85 30.48) (end 63.562 30.48) (width 0.25) (layer "F.Cu") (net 4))
 (segment (start 55.8 33.1501) (end 55.8 40.64) (width 0.25) (layer "F.Cu") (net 4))
 (segment (start 58.44 36.89) (end 58.44 50) (width 0.25) (layer "B.Cu") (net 36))
 (segment (start 43.18 21.63) (end 58.44 36.89) (width 0.25) (layer "B.Cu") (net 36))
 (segment (start 58.0281 24.13) (end 58.85 24.13) (width 0.25) (layer "F.Cu") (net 5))
 (segment (start 57.3861 24.772) (end 58.0281 24.13) (width 0.25) (layer "F.Cu") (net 5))
 (via (at 57.3861 24.772) (size 0.8) (drill 0.4) (layers "F.Cu" "B.Cu") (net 5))
 (segment (start 46.563 50.4594) (end 47.3617 51.2581) (width 0.25) (layer "B.Cu") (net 5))
 (segment (start 47.3617 51.2581) (end 59.6818 51.2581) (width 0.25) (layer "B.Cu") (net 5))
 (segment (start 59.6818 27.0677) (end 57.3861 24.772) (width 0.25) (layer "B.Cu") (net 5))
 (segment (start 46.563 50) (end 46.563 50.4594) (width 0.25) (layer "B.Cu") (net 5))
 (segment (start 59.6818 51.2581) (end 59.6818 27.0677) (width 0.25) (layer "B.Cu") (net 5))
 (segment (start 45.3379 50) (end 46.563 50) (width 0.25) (layer "B.Cu") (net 5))
 (segment (start 59.6818 51.2581) (end 61.4181 51.2581) (width 0.25) (layer "B.Cu") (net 5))
 (segment (start 61.4181 51.2581) (end 73.66 63.5) (width 0.25) (layer "B.Cu") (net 5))
 (segment (start 80.7874 27.0999) (end 80.7874 34.175) (width 0.25) (layer "F.Cu") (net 46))
 (segment (start 77.8175 24.13) (end 80.7874 27.0999) (width 0.25) (layer "F.Cu") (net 46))
 (segment (start 68.15 24.13) (end 77.8175 24.13) (width 0.25) (layer "F.Cu") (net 46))
 (segment (start 54.0024 60.96) (end 45.72 60.96) (width 0.25) (layer "F.Cu") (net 46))
 (segment (start 80.7874 34.175) (end 54.0024 60.96) (width 0.25) (layer "F.Cu") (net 46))
 (segment (start 58.85 22.86) (end 59.485 23.495) (width 0.25) (layer "F.Cu") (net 6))
 (segment (start 59.485 23.495) (end 77.8381 23.495) (width 0.25) (layer "F.Cu") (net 6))
 (segment (start 77.8381 23.495) (end 81.28 26.9369) (width 0.25) (layer "F.Cu") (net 6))
 (segment (start 81.28 26.9369) (end 81.28 63.5) (width 0.25) (layer "F.Cu") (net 6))
 (segment (start 52.005 27.305) (end 61.7555 27.305) (width 0.25) (layer "F.Cu") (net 1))
 (segment (start 80.3077 27.2569) (end 80.3077 33.9923) (width 0.25) (layer "F.Cu") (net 1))
 (segment (start 77.8158 24.765) (end 80.3077 27.2569) (width 0.25) (layer "F.Cu") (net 1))
 (segment (start 48.195 31.115) (end 52.005 27.305) (width 0.25) (layer "F.Cu") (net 1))
 (segment (start 64.2955 24.765) (end 77.8158 24.765) (width 0.25) (layer "F.Cu") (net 1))
 (segment (start 61.7555 27.305) (end 64.2955 24.765) (width 0.25) (layer "F.Cu") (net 1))
 (segment (start 80.3077 33.9923) (end 76.2 38.1) (width 0.25) (layer "F.Cu") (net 1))
 (segment (start 65.96 41.475) (end 65.96 38.86) (width 0.25) (layer "F.Cu") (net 37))
 (segment (start 65.96 38.86) (end 58.85 31.75) (width 0.25) (layer "F.Cu") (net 37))
 (segment (start 65.96 41.475) (end 77.3915 30.0435) (width 0.25) (layer "B.Cu") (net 37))
 (segment (start 77.3915 30.0435) (end 81.5165 30.0435) (width 0.25) (layer "B.Cu") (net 37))
 (segment (start 81.5165 30.0435) (end 83.62 27.94) (width 0.25) (layer "B.Cu") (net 37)))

